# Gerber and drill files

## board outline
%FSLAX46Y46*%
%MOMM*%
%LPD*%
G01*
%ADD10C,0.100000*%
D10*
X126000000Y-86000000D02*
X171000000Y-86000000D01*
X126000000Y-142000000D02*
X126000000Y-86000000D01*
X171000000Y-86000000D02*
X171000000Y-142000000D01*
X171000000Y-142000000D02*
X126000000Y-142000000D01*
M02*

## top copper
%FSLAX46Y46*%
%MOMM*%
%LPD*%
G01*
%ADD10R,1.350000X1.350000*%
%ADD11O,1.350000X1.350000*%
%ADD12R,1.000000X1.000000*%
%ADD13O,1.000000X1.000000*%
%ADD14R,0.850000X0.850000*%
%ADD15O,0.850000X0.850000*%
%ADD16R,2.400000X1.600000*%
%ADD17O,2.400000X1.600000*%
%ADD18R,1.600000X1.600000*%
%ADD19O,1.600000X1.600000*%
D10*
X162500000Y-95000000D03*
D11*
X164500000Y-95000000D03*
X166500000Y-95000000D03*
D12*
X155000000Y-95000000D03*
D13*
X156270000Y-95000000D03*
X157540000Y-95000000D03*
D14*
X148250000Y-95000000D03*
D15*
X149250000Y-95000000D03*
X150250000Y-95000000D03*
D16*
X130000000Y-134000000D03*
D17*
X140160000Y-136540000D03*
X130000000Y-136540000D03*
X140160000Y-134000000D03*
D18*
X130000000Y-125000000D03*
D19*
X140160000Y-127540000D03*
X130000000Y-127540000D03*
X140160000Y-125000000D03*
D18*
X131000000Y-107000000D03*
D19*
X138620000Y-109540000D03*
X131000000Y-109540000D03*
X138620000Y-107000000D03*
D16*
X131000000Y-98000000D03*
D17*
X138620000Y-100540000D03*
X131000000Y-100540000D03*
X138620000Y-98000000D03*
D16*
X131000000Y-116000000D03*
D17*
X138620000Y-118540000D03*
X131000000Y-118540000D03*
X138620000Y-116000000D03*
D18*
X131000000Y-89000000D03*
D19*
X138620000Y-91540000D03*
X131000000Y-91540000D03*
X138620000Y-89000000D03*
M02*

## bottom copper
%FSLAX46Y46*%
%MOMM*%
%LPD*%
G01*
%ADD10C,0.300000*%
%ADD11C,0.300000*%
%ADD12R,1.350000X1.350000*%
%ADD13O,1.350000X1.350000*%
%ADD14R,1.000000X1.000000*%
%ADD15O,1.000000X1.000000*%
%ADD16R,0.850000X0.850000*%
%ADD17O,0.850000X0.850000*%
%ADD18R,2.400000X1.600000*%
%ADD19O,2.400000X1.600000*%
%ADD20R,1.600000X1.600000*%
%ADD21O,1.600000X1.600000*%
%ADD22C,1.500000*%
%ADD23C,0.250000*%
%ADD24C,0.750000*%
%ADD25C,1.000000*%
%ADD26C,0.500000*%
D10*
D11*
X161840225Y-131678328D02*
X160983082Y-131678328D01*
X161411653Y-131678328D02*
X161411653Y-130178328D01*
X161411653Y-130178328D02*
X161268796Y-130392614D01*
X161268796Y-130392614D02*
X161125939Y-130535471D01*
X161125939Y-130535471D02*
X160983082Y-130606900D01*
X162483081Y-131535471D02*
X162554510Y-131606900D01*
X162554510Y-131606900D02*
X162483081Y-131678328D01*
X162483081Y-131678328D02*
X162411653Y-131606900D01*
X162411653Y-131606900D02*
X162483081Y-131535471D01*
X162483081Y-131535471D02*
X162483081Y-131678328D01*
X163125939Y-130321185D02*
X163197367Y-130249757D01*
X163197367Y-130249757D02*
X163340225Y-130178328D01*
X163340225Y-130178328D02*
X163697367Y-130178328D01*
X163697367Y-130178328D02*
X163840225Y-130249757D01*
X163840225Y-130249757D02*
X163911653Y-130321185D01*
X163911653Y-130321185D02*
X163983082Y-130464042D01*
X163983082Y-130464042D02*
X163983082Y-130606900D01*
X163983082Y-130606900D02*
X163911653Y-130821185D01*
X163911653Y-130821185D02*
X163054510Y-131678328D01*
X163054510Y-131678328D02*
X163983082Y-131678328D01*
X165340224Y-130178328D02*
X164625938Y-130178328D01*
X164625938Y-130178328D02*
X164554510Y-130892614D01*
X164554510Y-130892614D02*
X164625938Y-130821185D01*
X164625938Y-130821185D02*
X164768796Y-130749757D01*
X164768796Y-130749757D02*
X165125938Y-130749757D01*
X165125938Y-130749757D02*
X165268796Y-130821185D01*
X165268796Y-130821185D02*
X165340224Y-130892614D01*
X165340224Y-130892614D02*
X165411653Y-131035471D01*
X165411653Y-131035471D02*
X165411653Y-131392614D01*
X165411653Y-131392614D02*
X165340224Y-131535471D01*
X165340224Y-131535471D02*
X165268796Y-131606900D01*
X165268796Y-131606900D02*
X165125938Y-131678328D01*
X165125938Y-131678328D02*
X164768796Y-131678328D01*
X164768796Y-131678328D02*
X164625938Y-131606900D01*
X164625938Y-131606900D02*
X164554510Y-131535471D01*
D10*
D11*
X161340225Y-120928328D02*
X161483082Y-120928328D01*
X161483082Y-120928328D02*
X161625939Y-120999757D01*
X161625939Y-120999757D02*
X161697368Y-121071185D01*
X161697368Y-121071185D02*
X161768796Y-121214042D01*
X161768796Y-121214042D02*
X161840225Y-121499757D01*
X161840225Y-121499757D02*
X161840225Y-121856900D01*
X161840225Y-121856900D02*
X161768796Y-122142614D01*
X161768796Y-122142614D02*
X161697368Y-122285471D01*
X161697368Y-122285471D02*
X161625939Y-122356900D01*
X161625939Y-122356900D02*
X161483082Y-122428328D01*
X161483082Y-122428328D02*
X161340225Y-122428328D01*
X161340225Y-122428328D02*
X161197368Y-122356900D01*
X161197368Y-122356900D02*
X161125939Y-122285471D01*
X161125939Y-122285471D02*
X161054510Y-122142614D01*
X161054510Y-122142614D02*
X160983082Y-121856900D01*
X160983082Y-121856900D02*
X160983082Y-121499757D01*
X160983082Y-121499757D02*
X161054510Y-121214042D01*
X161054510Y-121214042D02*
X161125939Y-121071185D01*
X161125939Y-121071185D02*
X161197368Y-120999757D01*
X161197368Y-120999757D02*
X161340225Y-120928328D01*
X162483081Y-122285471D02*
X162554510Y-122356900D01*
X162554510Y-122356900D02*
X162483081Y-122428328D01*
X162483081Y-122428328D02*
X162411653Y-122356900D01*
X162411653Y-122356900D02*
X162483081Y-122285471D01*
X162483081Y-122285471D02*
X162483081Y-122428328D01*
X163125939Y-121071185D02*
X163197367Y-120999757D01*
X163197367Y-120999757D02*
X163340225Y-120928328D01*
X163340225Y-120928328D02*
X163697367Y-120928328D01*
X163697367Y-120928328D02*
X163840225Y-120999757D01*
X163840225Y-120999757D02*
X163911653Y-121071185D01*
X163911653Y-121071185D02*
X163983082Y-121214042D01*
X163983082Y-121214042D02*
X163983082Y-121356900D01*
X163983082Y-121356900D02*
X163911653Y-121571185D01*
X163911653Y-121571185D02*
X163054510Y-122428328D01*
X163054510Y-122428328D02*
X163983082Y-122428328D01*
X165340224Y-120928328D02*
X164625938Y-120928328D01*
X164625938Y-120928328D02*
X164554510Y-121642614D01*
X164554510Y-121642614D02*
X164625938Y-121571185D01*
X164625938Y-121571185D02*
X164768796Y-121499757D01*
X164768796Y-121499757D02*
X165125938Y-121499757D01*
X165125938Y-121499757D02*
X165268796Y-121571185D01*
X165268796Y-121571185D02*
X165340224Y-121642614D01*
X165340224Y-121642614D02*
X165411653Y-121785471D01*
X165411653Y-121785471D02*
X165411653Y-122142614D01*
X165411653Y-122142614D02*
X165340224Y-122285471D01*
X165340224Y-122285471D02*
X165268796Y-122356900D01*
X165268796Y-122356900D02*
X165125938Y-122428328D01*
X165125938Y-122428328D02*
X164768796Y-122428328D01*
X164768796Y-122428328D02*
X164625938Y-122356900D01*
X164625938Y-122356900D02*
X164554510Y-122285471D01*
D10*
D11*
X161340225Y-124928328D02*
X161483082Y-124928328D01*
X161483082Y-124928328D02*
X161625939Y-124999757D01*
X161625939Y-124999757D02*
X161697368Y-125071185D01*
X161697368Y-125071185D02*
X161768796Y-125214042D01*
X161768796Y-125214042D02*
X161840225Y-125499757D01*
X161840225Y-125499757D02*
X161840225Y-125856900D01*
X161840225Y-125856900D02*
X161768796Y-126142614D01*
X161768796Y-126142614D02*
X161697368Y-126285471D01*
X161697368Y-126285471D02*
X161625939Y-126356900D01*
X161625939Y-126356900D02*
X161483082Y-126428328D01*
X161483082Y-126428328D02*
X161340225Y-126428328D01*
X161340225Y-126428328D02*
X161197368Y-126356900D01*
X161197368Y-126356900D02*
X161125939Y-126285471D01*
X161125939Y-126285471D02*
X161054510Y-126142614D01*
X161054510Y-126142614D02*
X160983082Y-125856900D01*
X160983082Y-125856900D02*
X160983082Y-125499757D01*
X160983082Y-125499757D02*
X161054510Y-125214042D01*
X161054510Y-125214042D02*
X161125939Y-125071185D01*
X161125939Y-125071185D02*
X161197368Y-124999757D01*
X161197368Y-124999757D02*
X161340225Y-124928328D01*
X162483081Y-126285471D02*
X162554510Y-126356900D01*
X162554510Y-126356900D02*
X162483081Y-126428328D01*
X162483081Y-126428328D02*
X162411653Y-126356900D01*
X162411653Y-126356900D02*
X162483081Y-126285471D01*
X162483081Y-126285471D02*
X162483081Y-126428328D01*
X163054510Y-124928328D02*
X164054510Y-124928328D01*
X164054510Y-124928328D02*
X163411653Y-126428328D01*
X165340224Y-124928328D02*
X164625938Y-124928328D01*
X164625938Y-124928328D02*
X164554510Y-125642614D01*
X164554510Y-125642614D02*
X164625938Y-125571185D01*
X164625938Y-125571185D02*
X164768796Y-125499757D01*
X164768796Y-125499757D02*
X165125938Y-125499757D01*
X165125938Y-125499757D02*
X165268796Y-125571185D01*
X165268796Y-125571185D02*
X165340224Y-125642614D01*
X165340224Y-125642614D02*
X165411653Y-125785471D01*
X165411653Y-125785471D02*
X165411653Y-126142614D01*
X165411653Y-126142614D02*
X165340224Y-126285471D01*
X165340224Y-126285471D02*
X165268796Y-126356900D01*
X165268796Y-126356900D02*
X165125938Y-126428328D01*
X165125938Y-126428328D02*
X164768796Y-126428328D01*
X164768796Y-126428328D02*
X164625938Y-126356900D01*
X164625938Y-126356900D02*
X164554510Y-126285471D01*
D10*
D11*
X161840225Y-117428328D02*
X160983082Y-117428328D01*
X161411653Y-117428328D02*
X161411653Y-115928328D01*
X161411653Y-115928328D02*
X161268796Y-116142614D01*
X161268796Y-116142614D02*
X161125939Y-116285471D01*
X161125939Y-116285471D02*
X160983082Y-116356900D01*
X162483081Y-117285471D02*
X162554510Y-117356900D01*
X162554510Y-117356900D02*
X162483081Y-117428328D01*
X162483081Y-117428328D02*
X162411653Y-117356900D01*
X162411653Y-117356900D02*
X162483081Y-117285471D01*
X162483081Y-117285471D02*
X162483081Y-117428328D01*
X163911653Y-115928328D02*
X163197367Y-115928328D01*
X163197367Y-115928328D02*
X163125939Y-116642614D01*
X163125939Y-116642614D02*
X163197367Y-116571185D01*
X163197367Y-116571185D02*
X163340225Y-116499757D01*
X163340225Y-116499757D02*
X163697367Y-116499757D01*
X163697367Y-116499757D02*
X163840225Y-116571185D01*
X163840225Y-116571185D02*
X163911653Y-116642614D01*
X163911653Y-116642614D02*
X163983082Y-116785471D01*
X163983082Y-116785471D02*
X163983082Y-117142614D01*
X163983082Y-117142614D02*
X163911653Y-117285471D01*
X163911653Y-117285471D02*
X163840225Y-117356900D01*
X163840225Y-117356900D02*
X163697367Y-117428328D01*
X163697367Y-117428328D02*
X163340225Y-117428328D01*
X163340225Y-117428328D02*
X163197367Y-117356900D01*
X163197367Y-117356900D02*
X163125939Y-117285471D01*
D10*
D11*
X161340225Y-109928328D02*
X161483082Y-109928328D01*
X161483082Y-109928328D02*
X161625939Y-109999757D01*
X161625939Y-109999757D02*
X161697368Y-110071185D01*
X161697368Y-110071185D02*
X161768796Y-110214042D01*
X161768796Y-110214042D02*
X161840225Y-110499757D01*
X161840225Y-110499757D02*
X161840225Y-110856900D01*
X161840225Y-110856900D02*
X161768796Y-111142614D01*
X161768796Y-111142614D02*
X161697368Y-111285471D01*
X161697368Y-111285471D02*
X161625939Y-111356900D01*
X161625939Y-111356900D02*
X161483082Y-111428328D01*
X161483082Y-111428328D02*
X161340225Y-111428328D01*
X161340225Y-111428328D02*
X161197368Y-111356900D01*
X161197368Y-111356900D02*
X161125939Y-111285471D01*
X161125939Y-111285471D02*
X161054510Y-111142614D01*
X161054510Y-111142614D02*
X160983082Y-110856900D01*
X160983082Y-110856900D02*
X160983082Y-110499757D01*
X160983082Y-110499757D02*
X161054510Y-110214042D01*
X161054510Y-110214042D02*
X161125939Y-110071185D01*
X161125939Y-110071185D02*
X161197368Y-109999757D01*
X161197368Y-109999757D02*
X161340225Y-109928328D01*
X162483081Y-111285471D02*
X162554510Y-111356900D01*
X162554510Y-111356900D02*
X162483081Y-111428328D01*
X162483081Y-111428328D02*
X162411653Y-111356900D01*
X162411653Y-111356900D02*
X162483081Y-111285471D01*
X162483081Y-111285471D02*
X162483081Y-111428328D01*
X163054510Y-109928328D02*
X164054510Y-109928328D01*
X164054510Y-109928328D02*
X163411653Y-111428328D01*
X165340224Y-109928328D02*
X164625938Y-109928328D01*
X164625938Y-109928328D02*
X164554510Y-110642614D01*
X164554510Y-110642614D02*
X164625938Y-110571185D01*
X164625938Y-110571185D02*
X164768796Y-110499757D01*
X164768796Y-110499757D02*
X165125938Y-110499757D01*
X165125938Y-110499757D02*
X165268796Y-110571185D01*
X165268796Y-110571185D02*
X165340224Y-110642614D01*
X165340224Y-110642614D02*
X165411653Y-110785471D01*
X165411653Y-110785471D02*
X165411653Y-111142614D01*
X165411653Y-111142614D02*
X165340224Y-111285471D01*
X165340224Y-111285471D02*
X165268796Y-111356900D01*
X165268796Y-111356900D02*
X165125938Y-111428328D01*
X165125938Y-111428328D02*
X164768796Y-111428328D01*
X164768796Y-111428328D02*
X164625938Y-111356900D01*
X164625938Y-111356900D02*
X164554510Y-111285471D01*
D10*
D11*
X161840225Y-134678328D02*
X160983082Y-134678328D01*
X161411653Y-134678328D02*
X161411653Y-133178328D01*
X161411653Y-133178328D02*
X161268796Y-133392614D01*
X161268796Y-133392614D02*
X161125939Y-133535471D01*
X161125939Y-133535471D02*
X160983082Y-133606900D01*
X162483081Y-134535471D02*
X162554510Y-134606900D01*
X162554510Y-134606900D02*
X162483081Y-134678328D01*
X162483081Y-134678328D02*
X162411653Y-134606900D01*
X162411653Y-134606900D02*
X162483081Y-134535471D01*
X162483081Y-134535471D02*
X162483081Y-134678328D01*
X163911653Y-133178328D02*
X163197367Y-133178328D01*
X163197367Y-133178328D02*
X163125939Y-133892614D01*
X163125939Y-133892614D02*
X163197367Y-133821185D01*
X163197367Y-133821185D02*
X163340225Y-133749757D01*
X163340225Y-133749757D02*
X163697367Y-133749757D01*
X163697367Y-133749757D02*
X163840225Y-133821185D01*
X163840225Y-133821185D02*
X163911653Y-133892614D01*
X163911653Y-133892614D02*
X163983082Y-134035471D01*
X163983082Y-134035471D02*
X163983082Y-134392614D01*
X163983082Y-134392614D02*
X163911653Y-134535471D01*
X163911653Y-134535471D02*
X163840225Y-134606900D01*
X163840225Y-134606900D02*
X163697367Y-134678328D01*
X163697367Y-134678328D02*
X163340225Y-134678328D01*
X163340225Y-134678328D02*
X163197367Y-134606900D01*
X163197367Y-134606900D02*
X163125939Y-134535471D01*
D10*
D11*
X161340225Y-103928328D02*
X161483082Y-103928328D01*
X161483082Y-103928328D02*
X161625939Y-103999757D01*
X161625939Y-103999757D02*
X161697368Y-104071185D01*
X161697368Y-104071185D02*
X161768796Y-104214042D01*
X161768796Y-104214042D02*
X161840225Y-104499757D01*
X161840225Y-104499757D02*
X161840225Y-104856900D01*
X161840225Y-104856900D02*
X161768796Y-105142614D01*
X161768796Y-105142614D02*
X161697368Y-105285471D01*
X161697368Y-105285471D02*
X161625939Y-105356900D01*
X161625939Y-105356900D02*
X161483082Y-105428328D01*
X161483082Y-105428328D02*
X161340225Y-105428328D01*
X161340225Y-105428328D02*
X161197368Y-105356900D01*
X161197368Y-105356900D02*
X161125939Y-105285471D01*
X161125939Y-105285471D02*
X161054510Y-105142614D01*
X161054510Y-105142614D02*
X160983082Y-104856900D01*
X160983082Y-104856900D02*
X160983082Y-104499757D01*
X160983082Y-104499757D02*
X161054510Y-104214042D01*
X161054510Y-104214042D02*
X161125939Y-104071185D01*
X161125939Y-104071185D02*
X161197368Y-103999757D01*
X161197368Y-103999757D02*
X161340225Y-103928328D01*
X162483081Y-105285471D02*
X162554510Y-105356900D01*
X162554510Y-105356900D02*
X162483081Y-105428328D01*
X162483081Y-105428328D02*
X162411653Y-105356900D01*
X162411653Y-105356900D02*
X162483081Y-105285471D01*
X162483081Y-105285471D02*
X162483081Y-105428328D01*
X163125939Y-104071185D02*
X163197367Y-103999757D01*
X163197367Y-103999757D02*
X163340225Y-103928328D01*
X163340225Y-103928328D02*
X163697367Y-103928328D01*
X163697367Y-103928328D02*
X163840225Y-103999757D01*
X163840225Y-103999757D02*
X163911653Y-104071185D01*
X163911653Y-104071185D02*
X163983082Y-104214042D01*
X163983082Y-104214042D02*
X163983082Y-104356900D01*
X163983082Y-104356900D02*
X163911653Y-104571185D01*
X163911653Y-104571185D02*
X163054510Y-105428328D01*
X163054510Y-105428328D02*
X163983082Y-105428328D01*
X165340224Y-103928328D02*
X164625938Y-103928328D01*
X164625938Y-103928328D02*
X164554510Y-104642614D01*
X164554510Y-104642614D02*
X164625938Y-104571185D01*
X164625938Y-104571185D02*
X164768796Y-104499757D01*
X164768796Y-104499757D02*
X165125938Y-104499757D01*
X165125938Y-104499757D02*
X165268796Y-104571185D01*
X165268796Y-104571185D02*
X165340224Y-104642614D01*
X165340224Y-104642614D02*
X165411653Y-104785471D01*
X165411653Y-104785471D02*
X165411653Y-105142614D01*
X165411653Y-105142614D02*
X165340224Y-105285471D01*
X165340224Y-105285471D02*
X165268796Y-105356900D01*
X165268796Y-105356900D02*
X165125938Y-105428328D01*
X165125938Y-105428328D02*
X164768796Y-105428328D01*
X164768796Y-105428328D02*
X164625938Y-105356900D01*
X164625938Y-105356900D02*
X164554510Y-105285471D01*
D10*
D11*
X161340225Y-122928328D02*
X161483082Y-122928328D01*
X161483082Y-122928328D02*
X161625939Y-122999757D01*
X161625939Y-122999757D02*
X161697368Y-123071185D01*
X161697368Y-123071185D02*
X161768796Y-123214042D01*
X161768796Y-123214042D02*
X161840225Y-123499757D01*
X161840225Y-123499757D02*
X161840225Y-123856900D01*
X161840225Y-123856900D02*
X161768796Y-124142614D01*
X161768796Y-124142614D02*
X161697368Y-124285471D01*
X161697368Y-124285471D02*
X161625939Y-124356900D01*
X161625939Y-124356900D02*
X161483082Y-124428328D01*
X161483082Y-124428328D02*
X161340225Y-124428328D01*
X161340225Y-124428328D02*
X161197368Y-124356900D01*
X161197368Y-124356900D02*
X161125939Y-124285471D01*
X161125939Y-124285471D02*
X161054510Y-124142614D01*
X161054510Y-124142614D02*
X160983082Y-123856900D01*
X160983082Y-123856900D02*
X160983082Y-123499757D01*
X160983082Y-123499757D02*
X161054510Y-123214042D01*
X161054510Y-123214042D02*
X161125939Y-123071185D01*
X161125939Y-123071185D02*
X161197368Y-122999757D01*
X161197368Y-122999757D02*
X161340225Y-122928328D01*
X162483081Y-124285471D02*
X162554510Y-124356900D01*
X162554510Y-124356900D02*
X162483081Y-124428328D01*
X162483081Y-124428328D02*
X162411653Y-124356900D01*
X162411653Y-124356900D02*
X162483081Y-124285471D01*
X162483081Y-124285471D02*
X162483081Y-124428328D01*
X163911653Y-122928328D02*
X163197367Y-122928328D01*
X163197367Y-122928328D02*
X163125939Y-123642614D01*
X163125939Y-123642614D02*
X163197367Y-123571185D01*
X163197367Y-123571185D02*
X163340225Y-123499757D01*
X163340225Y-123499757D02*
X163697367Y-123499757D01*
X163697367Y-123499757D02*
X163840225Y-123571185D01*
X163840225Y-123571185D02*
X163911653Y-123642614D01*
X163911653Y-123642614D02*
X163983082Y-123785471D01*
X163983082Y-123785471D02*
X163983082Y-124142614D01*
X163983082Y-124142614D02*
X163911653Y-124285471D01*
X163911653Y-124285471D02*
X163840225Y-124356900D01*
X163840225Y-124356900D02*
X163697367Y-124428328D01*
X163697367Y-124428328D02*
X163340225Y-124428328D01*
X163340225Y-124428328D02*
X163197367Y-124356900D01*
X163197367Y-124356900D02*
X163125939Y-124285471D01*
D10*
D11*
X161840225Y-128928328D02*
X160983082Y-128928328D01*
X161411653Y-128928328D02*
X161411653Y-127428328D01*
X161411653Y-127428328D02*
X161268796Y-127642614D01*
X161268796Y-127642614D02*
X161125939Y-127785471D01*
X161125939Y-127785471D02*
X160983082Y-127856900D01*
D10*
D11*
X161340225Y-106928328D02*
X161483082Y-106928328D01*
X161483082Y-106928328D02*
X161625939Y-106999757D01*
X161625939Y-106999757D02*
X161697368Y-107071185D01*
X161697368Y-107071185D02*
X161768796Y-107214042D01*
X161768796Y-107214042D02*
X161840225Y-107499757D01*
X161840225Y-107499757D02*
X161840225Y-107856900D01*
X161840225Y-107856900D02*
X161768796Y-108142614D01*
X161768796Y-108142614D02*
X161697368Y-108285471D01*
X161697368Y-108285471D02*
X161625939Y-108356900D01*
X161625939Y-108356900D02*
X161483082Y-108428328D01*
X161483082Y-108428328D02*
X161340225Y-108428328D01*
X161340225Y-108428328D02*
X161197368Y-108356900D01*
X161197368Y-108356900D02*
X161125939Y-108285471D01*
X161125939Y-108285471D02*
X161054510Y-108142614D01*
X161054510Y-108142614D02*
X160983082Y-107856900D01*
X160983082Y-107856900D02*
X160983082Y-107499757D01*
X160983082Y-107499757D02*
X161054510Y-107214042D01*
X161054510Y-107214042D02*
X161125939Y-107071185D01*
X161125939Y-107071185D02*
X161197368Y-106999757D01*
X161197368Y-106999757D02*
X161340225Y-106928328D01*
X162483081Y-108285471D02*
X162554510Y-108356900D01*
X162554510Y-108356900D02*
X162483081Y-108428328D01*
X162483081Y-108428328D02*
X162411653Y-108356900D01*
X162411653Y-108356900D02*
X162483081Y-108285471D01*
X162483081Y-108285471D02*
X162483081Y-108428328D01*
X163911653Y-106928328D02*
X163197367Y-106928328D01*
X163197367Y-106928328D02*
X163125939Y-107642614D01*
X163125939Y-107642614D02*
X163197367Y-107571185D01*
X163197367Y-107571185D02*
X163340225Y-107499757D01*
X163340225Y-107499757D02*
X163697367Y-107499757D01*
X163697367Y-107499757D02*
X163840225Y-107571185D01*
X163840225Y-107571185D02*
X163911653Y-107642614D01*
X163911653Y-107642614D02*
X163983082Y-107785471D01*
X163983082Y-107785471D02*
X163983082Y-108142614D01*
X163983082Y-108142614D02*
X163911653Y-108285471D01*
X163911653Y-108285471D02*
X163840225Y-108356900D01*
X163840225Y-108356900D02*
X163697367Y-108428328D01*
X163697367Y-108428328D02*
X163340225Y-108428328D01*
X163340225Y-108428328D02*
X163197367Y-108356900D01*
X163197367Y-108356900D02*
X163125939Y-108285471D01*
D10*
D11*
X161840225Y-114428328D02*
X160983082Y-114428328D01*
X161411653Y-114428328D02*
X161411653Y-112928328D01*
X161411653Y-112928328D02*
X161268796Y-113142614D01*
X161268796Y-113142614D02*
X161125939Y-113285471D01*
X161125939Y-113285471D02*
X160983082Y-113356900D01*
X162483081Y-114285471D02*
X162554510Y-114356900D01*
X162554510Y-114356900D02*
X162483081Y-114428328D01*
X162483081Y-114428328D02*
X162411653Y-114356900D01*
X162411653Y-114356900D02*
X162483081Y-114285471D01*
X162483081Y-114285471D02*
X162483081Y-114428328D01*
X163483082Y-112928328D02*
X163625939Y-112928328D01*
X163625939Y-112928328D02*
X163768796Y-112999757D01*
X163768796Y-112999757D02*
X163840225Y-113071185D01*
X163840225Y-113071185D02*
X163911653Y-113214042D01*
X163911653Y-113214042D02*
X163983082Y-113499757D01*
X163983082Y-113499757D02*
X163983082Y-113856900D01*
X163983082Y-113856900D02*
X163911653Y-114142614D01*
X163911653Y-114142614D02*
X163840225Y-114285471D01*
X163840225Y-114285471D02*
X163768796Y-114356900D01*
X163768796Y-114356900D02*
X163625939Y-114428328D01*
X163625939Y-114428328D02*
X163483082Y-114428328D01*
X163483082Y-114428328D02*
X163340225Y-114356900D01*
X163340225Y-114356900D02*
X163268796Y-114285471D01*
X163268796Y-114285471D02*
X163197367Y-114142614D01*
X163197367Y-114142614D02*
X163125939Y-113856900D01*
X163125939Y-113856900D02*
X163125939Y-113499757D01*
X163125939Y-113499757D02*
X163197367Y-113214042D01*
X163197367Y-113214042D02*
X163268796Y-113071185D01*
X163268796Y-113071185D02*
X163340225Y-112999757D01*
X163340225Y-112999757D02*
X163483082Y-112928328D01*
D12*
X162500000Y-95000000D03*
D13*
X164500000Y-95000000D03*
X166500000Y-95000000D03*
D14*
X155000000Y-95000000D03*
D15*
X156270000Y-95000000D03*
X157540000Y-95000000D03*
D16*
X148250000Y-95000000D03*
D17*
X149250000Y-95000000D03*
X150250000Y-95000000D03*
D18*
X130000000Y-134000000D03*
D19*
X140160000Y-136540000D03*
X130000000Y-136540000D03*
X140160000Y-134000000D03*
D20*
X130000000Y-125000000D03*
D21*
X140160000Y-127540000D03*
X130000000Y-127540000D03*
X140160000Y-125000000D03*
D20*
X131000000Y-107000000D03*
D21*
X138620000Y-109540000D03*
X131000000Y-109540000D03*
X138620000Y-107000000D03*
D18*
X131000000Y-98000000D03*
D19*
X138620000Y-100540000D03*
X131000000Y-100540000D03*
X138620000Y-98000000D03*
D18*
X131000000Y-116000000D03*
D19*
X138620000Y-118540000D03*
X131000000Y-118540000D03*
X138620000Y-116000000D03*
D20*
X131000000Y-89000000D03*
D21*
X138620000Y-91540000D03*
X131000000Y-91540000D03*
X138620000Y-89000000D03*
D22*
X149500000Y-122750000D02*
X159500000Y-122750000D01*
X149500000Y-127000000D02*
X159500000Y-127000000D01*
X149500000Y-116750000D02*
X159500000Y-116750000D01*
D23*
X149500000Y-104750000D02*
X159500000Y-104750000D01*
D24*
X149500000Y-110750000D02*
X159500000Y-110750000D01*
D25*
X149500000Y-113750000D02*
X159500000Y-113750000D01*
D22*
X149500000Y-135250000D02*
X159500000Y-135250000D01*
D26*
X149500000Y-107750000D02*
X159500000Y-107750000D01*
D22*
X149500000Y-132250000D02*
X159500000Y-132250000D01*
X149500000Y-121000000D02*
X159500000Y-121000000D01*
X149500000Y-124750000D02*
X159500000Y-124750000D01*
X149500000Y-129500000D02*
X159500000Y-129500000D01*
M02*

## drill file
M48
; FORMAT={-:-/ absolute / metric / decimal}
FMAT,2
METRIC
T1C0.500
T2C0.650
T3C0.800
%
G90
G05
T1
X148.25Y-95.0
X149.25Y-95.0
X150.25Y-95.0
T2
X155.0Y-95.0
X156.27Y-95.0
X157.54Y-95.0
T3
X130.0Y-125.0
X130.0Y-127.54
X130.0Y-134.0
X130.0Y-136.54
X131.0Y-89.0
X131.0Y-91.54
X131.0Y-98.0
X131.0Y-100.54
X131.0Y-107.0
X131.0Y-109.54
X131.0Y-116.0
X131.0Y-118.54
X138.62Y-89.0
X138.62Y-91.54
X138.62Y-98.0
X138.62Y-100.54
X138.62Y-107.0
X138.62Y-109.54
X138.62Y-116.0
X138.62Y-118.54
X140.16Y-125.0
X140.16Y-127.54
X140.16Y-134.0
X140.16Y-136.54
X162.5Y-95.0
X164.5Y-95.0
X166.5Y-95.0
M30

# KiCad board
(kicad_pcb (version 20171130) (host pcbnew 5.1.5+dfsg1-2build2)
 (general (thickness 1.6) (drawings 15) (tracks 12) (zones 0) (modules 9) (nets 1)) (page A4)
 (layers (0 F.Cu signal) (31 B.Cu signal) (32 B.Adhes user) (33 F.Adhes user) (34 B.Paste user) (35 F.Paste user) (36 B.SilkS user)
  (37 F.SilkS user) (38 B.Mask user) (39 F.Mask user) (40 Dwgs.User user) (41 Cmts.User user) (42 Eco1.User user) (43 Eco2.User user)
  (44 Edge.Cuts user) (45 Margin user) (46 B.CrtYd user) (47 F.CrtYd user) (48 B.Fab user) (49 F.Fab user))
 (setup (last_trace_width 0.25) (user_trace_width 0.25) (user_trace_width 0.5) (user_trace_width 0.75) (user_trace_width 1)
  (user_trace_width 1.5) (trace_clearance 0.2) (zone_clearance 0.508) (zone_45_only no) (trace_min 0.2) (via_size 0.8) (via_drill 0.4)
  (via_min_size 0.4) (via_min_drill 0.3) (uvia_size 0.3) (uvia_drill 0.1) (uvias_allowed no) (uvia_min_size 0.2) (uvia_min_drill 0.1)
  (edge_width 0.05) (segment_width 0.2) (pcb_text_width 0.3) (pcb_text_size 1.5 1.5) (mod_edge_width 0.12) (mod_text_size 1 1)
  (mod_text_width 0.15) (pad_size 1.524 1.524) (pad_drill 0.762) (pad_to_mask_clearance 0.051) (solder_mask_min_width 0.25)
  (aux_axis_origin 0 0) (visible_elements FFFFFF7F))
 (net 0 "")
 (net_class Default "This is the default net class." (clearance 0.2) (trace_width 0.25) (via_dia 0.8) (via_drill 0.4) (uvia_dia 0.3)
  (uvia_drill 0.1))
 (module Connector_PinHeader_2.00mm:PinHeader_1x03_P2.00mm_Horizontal (layer F.Cu) (at 162.5 95 90)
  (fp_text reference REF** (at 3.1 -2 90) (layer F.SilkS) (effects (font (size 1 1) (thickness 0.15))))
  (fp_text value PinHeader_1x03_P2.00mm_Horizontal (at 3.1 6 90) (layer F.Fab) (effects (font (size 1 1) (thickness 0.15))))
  (pad 1 thru_hole rect (at 0 0 90) (size 1.35 1.35) (drill 0.8) (layers *.Cu *.Mask))
  (pad 2 thru_hole oval (at 0 2 90) (size 1.35 1.35) (drill 0.8) (layers *.Cu *.Mask))
  (pad 3 thru_hole oval (at 0 4 90) (size 1.35 1.35) (drill 0.8) (layers *.Cu *.Mask)))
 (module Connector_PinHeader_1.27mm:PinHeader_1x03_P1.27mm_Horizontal (layer F.Cu) (at 155 95 90)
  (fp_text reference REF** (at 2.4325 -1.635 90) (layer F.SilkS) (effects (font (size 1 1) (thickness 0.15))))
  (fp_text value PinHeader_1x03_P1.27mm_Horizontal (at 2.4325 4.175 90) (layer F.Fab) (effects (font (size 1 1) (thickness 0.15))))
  (pad 1 thru_hole rect (at 0 0 90) (size 1 1) (drill 0.65) (layers *.Cu *.Mask))
  (pad 2 thru_hole oval (at 0 1.27 90) (size 1 1) (drill 0.65) (layers *.Cu *.Mask))
  (pad 3 thru_hole oval (at 0 2.54 90) (size 1 1) (drill 0.65) (layers *.Cu *.Mask)))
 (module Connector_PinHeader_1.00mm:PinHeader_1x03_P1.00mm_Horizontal (layer F.Cu) (at 148.25 95 90)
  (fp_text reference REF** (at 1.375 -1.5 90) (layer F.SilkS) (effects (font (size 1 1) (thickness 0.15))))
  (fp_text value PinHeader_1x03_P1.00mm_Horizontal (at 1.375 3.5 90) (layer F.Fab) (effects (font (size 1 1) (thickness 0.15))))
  (pad 1 thru_hole rect (at 0 0 90) (size 0.85 0.85) (drill 0.5) (layers *.Cu *.Mask))
  (pad 2 thru_hole oval (at 0 1 90) (size 0.85 0.85) (drill 0.5) (layers *.Cu *.Mask))
  (pad 3 thru_hole oval (at 0 2 90) (size 0.85 0.85) (drill 0.5) (layers *.Cu *.Mask)))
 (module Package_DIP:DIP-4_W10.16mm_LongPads (layer F.Cu) (at 130 134)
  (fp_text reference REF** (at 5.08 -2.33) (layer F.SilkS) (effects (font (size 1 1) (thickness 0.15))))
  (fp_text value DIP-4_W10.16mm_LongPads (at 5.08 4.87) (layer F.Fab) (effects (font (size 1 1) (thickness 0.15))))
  (pad 1 thru_hole rect (at 0 0) (size 2.4 1.6) (drill 0.8) (layers *.Cu *.Mask))
  (pad 3 thru_hole oval (at 10.16 2.54) (size 2.4 1.6) (drill 0.8) (layers *.Cu *.Mask))
  (pad 2 thru_hole oval (at 0 2.54) (size 2.4 1.6) (drill 0.8) (layers *.Cu *.Mask))
  (pad 4 thru_hole oval (at 10.16 0) (size 2.4 1.6) (drill 0.8) (layers *.Cu *.Mask)))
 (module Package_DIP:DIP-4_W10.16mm (layer F.Cu) (at 130 125)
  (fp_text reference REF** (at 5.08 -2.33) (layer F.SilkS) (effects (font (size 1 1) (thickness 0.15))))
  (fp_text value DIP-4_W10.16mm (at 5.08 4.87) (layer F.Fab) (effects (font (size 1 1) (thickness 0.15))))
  (pad 1 thru_hole rect (at 0 0) (size 1.6 1.6) (drill 0.8) (layers *.Cu *.Mask))
  (pad 3 thru_hole oval (at 10.16 2.54) (size 1.6 1.6) (drill 0.8) (layers *.Cu *.Mask))
  (pad 2 thru_hole oval (at 0 2.54) (size 1.6 1.6) (drill 0.8) (layers *.Cu *.Mask))
  (pad 4 thru_hole oval (at 10.16 0) (size 1.6 1.6) (drill 0.8) (layers *.Cu *.Mask)))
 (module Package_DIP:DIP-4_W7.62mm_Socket (layer F.Cu) (at 131 107)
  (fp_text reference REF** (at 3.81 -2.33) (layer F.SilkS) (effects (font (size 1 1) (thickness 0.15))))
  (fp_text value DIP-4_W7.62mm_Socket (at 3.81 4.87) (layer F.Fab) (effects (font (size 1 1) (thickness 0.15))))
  (pad 1 thru_hole rect (at 0 0) (size 1.6 1.6) (drill 0.8) (layers *.Cu *.Mask))
  (pad 3 thru_hole oval (at 7.62 2.54) (size 1.6 1.6) (drill 0.8) (layers *.Cu *.Mask))
  (pad 2 thru_hole oval (at 0 2.54) (size 1.6 1.6) (drill 0.8) (layers *.Cu *.Mask))
  (pad 4 thru_hole oval (at 7.62 0) (size 1.6 1.6) (drill 0.8) (layers *.Cu *.Mask)))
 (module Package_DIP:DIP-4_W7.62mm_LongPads (layer F.Cu) (at 131 98)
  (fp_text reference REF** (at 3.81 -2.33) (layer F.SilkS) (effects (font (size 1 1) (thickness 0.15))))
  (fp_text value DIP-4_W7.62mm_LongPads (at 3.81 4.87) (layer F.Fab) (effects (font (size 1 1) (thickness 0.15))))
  (pad 1 thru_hole rect (at 0 0) (size 2.4 1.6) (drill 0.8) (layers *.Cu *.Mask))
  (pad 3 thru_hole oval (at 7.62 2.54) (size 2.4 1.6) (drill 0.8) (layers *.Cu *.Mask))
  (pad 2 thru_hole oval (at 0 2.54) (size 2.4 1.6) (drill 0.8) (layers *.Cu *.Mask))
  (pad 4 thru_hole oval (at 7.62 0) (size 2.4 1.6) (drill 0.8) (layers *.Cu *.Mask)))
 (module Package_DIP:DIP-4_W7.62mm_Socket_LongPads (layer F.Cu) (at 131 116)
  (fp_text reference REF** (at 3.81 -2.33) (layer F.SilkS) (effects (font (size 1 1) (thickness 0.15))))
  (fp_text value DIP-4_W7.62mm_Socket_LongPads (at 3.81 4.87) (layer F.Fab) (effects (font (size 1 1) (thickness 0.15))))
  (pad 1 thru_hole rect (at 0 0) (size 2.4 1.6) (drill 0.8) (layers *.Cu *.Mask))
  (pad 3 thru_hole oval (at 7.62 2.54) (size 2.4 1.6) (drill 0.8) (layers *.Cu *.Mask))
  (pad 2 thru_hole oval (at 0 2.54) (size 2.4 1.6) (drill 0.8) (layers *.Cu *.Mask))
  (pad 4 thru_hole oval (at 7.62 0) (size 2.4 1.6) (drill 0.8) (layers *.Cu *.Mask)))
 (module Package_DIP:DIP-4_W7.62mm (layer F.Cu) (at 131 89)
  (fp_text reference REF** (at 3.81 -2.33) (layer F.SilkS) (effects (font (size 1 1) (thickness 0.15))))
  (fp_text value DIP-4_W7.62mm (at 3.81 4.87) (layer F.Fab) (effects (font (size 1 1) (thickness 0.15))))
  (pad 1 thru_hole rect (at 0 0) (size 1.6 1.6) (drill 0.8) (layers *.Cu *.Mask))
  (pad 3 thru_hole oval (at 7.62 2.54) (size 1.6 1.6) (drill 0.8) (layers *.Cu *.Mask))
  (pad 2 thru_hole oval (at 0 2.54) (size 1.6 1.6) (drill 0.8) (layers *.Cu *.Mask))
  (pad 4 thru_hole oval (at 7.62 0) (size 1.6 1.6) (drill 0.8) (layers *.Cu *.Mask)))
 (gr_line (start 126 86) (end 171 86) (layer Edge.Cuts) (width 0.1))
 (gr_line (start 126 142) (end 126 86) (layer Edge.Cuts) (width 0.1))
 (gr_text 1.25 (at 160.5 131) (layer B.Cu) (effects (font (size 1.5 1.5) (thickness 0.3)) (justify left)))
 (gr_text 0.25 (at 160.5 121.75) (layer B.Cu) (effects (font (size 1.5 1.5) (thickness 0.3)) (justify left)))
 (gr_line (start 171 86) (end 171 142) (layer Edge.Cuts) (width 0.1))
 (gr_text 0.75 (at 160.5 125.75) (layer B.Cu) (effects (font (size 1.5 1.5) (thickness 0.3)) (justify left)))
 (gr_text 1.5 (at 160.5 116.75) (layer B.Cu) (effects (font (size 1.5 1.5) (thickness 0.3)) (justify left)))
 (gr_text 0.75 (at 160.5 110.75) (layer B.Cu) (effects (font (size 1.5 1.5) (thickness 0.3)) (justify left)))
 (gr_line (start 171 142) (end 126 142) (layer Edge.Cuts) (width 0.1))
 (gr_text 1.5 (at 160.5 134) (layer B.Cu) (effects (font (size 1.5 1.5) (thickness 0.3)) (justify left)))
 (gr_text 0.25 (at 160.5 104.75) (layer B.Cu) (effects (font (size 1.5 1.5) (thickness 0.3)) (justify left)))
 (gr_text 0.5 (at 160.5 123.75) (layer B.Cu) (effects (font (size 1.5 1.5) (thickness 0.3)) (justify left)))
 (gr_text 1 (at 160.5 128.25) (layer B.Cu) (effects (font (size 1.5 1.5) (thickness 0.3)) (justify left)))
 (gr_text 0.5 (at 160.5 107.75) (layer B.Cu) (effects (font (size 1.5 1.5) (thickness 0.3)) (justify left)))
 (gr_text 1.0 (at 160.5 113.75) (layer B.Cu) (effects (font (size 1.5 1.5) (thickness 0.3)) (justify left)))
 (segment (start 149.5 122.75) (end 159.5 122.75) (width 1.5) (layer B.Cu) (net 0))
 (segment (start 149.5 127) (end 159.5 127) (width 1.5) (layer B.Cu) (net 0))
 (segment (start 149.5 116.75) (end 159.5 116.75) (width 1.5) (layer B.Cu) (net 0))
 (segment (start 149.5 104.75) (end 159.5 104.75) (width 0.25) (layer B.Cu) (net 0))
 (segment (start 149.5 110.75) (end 159.5 110.75) (width 0.75) (layer B.Cu) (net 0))
 (segment (start 149.5 113.75) (end 159.5 113.75) (width 1) (layer B.Cu) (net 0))
 (segment (start 149.5 135.25) (end 159.5 135.25) (width 1.5) (layer B.Cu) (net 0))
 (segment (start 149.5 107.75) (end 159.5 107.75) (width 0.5) (layer B.Cu) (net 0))
 (segment (start 149.5 132.25) (end 159.5 132.25) (width 1.5) (layer B.Cu) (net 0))
 (segment (start 149.5 121) (end 159.5 121) (width 1.5) (layer B.Cu) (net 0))
 (segment (start 149.5 124.75) (end 159.5 124.75) (width 1.5) (layer B.Cu) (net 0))
 (segment (start 149.5 129.5) (end 159.5 129.5) (width 1.5) (layer B.Cu) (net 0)))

